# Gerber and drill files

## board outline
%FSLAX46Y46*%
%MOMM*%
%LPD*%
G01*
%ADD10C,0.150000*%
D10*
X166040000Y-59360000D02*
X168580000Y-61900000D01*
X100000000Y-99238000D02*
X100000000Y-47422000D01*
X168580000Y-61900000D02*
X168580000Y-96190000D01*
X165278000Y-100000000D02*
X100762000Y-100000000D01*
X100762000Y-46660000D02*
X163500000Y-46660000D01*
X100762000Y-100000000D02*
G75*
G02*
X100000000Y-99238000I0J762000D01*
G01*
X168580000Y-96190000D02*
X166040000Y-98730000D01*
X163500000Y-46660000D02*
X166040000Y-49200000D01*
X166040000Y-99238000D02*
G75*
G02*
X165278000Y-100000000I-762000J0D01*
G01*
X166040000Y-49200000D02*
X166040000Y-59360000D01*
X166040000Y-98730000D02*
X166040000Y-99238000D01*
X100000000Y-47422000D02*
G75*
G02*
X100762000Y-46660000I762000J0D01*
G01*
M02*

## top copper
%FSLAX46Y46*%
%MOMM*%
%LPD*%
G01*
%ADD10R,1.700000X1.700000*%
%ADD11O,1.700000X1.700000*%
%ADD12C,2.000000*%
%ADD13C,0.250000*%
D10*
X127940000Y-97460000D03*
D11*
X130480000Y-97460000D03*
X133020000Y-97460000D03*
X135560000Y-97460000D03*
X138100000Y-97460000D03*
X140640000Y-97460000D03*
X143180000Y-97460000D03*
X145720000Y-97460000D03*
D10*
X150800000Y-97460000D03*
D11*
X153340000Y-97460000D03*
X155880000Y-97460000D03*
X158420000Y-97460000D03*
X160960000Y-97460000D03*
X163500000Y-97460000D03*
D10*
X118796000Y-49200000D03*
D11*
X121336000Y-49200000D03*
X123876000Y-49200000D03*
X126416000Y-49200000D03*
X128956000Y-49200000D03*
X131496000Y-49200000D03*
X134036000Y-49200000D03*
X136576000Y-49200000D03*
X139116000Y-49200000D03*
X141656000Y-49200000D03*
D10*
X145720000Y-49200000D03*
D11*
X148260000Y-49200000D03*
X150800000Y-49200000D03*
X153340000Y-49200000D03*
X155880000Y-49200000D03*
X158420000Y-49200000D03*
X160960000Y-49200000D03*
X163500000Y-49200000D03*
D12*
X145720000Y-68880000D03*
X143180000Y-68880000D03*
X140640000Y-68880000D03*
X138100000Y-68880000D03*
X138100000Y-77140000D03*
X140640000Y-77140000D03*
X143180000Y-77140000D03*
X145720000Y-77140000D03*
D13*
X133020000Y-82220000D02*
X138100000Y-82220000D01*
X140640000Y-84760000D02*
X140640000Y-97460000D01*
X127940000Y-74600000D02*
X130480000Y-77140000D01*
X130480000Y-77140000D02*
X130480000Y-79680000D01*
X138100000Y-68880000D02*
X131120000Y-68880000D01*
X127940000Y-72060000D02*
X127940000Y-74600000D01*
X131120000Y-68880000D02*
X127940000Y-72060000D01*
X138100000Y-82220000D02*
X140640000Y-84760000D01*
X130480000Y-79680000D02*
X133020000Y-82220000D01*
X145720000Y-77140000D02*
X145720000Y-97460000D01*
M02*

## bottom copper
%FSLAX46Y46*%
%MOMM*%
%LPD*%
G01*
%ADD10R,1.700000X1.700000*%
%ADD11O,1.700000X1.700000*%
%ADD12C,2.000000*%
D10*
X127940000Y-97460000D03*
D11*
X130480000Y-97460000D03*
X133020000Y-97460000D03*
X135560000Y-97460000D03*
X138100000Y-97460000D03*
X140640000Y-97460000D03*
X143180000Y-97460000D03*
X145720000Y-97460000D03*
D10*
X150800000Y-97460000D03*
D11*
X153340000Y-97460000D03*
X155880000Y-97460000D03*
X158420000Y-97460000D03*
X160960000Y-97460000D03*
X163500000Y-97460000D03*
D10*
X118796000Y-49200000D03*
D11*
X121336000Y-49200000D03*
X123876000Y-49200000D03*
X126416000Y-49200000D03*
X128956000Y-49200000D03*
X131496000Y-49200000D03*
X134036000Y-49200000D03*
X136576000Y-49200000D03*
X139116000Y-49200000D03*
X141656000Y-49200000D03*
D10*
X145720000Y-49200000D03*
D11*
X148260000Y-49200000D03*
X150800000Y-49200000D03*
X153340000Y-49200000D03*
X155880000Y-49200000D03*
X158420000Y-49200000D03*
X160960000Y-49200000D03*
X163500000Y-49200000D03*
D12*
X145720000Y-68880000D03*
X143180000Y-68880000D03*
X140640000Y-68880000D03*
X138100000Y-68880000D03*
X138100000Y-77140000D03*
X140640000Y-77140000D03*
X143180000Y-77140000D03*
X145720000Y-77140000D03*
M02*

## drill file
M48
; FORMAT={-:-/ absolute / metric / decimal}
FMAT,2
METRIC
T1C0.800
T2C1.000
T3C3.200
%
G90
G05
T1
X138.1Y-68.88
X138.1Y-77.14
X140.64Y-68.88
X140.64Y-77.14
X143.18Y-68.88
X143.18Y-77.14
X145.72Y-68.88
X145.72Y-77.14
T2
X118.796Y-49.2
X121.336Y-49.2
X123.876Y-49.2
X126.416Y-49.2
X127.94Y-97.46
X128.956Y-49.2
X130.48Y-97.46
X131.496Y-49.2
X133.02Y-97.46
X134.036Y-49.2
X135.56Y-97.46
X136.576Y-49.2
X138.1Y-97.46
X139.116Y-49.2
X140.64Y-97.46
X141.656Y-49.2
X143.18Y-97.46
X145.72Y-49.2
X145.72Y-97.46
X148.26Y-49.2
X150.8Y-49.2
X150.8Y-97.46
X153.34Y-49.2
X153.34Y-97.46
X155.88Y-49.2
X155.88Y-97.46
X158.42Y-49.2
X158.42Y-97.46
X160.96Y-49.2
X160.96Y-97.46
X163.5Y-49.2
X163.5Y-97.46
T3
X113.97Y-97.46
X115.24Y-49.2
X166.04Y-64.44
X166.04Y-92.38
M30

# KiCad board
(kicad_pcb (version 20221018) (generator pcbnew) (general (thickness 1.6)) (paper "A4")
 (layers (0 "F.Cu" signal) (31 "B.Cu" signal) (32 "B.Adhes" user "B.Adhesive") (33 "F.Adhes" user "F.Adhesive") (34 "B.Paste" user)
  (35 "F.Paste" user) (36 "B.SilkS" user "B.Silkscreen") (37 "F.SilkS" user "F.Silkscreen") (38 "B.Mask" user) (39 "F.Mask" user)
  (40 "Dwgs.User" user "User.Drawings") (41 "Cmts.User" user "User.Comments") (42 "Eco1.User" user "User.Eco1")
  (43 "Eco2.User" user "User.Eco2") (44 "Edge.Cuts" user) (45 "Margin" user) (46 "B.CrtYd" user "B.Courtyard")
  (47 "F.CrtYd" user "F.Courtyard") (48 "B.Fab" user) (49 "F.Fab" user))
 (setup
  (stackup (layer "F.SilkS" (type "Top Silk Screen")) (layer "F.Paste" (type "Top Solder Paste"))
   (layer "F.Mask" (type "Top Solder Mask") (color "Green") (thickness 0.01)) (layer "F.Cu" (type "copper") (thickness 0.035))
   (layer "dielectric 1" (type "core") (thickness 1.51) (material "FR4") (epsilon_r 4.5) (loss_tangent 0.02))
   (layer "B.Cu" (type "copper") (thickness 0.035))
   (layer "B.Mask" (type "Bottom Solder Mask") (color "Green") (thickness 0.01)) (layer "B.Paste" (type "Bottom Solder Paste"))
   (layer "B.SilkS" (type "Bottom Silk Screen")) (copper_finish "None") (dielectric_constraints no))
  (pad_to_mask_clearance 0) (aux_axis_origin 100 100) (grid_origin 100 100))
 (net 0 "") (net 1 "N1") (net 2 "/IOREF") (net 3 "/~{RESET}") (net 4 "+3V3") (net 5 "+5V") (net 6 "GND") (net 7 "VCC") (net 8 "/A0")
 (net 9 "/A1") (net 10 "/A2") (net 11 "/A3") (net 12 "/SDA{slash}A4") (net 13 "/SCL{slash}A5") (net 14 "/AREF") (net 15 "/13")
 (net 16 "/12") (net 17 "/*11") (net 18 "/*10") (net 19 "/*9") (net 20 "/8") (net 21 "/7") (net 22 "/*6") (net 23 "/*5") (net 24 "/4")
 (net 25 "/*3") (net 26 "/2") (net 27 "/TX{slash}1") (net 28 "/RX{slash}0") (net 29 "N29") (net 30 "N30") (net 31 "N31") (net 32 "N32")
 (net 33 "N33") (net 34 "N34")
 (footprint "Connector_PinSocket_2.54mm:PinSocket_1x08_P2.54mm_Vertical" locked (layer "F.Cu") (at 127.94 97.46 90)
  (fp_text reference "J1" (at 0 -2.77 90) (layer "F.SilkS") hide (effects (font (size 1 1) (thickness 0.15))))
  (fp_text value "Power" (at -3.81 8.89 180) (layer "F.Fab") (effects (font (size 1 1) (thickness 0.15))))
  (pad "1" thru_hole rect locked (at 0 0 90) (size 1.7 1.7) (drill 1) (layers "*.Cu" "*.Mask") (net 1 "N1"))
  (pad "2" thru_hole oval locked (at 0 2.54 90) (size 1.7 1.7) (drill 1) (layers "*.Cu" "*.Mask") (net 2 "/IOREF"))
  (pad "3" thru_hole oval locked (at 0 5.08 90) (size 1.7 1.7) (drill 1) (layers "*.Cu" "*.Mask") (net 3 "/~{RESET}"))
  (pad "4" thru_hole oval locked (at 0 7.62 90) (size 1.7 1.7) (drill 1) (layers "*.Cu" "*.Mask") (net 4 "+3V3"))
  (pad "5" thru_hole oval locked (at 0 10.16 90) (size 1.7 1.7) (drill 1) (layers "*.Cu" "*.Mask") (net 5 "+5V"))
  (pad "6" thru_hole oval locked (at 0 12.7 90) (size 1.7 1.7) (drill 1) (layers "*.Cu" "*.Mask") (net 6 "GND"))
  (pad "7" thru_hole oval locked (at 0 15.24 90) (size 1.7 1.7) (drill 1) (layers "*.Cu" "*.Mask") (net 6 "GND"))
  (pad "8" thru_hole oval locked (at 0 17.78 90) (size 1.7 1.7) (drill 1) (layers "*.Cu" "*.Mask") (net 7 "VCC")))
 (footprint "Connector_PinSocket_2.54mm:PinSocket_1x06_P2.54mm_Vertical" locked (layer "F.Cu") (at 150.8 97.46 90)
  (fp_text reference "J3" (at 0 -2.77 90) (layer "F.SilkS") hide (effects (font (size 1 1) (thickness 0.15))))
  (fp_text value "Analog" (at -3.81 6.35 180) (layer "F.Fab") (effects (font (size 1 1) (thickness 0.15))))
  (pad "1" thru_hole rect locked (at 0 0 90) (size 1.7 1.7) (drill 1) (layers "*.Cu" "*.Mask") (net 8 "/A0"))
  (pad "2" thru_hole oval locked (at 0 2.54 90) (size 1.7 1.7) (drill 1) (layers "*.Cu" "*.Mask") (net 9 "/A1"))
  (pad "3" thru_hole oval locked (at 0 5.08 90) (size 1.7 1.7) (drill 1) (layers "*.Cu" "*.Mask") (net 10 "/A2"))
  (pad "4" thru_hole oval locked (at 0 7.62 90) (size 1.7 1.7) (drill 1) (layers "*.Cu" "*.Mask") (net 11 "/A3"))
  (pad "5" thru_hole oval locked (at 0 10.16 90) (size 1.7 1.7) (drill 1) (layers "*.Cu" "*.Mask") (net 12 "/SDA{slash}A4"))
  (pad "6" thru_hole oval locked (at 0 12.7 90) (size 1.7 1.7) (drill 1) (layers "*.Cu" "*.Mask") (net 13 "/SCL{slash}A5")))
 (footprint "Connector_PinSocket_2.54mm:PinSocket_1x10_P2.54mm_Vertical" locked (layer "F.Cu") (at 118.796 49.2 90)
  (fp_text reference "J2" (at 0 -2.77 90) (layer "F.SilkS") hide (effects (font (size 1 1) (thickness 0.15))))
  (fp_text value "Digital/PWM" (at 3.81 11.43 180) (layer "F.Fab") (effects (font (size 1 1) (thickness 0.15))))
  (pad "1" thru_hole rect locked (at 0 0 90) (size 1.7 1.7) (drill 1) (layers "*.Cu" "*.Mask") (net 13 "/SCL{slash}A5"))
  (pad "2" thru_hole oval locked (at 0 2.54 90) (size 1.7 1.7) (drill 1) (layers "*.Cu" "*.Mask") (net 12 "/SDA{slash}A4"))
  (pad "3" thru_hole oval locked (at 0 5.08 90) (size 1.7 1.7) (drill 1) (layers "*.Cu" "*.Mask") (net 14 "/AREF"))
  (pad "4" thru_hole oval locked (at 0 7.62 90) (size 1.7 1.7) (drill 1) (layers "*.Cu" "*.Mask") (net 6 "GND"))
  (pad "5" thru_hole oval locked (at 0 10.16 90) (size 1.7 1.7) (drill 1) (layers "*.Cu" "*.Mask") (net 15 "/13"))
  (pad "6" thru_hole oval locked (at 0 12.7 90) (size 1.7 1.7) (drill 1) (layers "*.Cu" "*.Mask") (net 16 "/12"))
  (pad "7" thru_hole oval locked (at 0 15.24 90) (size 1.7 1.7) (drill 1) (layers "*.Cu" "*.Mask") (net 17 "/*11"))
  (pad "8" thru_hole oval locked (at 0 17.78 90) (size 1.7 1.7) (drill 1) (layers "*.Cu" "*.Mask") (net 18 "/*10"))
  (pad "9" thru_hole oval locked (at 0 20.32 90) (size 1.7 1.7) (drill 1) (layers "*.Cu" "*.Mask") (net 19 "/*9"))
  (pad "10" thru_hole oval locked (at 0 22.86 90) (size 1.7 1.7) (drill 1) (layers "*.Cu" "*.Mask") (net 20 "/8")))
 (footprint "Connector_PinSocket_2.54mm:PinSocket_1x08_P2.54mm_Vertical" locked (layer "F.Cu") (at 145.72 49.2 90)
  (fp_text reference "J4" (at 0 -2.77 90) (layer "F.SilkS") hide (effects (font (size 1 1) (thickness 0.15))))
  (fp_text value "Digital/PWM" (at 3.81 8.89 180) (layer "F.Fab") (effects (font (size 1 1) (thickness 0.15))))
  (pad "1" thru_hole rect locked (at 0 0 90) (size 1.7 1.7) (drill 1) (layers "*.Cu" "*.Mask") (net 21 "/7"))
  (pad "2" thru_hole oval locked (at 0 2.54 90) (size 1.7 1.7) (drill 1) (layers "*.Cu" "*.Mask") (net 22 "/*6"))
  (pad "3" thru_hole oval locked (at 0 5.08 90) (size 1.7 1.7) (drill 1) (layers "*.Cu" "*.Mask") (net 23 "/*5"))
  (pad "4" thru_hole oval locked (at 0 7.62 90) (size 1.7 1.7) (drill 1) (layers "*.Cu" "*.Mask") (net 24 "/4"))
  (pad "5" thru_hole oval locked (at 0 10.16 90) (size 1.7 1.7) (drill 1) (layers "*.Cu" "*.Mask") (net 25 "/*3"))
  (pad "6" thru_hole oval locked (at 0 12.7 90) (size 1.7 1.7) (drill 1) (layers "*.Cu" "*.Mask") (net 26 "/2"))
  (pad "7" thru_hole oval locked (at 0 15.24 90) (size 1.7 1.7) (drill 1) (layers "*.Cu" "*.Mask") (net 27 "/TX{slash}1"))
  (pad "8" thru_hole oval locked (at 0 17.78 90) (size 1.7 1.7) (drill 1) (layers "*.Cu" "*.Mask") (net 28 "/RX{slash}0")))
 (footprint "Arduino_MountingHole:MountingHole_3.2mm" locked (layer "F.Cu") (at 115.24 49.2)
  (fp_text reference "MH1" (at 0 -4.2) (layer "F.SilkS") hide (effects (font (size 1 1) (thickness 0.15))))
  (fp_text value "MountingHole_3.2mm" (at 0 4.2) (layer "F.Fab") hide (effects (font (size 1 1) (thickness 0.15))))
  (pad "" np_thru_hole circle locked (at 0 0) (size 3.2 3.2) (drill 3.2) (layers "*.Cu" "*.Mask")))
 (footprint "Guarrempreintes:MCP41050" (layer "F.Cu") (at 141.91 72.64 180)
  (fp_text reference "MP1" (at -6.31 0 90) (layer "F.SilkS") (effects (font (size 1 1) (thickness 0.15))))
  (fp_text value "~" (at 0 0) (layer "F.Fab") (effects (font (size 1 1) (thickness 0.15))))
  (pad "1" thru_hole circle (at -3.81 3.76 180) (size 2 2) (drill 0.8) (layers "*.Cu" "*.Mask") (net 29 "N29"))
  (pad "2" thru_hole circle (at -1.27 3.76 180) (size 2 2) (drill 0.8) (layers "*.Cu" "*.Mask") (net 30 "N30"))
  (pad "3" thru_hole circle (at 1.27 3.76 180) (size 2 2) (drill 0.8) (layers "*.Cu" "*.Mask") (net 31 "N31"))
  (pad "4" thru_hole circle (at 3.81 3.76 180) (size 2 2) (drill 0.8) (layers "*.Cu" "*.Mask") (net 6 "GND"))
  (pad "5" thru_hole circle (at 3.81 -4.5 180) (size 2 2) (drill 0.8) (layers "*.Cu" "*.Mask") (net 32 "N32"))
  (pad "6" thru_hole circle (at 1.27 -4.5 180) (size 2 2) (drill 0.8) (layers "*.Cu" "*.Mask") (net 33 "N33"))
  (pad "7" thru_hole circle (at -1.27 -4.5 180) (size 2 2) (drill 0.8) (layers "*.Cu" "*.Mask") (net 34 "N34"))
  (pad "8" thru_hole circle (at -3.81 -4.5 180) (size 2 2) (drill 0.8) (layers "*.Cu" "*.Mask") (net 7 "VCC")))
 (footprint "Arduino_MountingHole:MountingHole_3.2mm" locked (layer "F.Cu") (at 113.97 97.46)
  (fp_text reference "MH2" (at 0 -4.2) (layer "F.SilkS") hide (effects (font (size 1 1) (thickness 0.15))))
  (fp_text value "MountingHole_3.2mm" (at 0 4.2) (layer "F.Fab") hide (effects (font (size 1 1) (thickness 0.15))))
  (pad "" np_thru_hole circle locked (at 0 0) (size 3.2 3.2) (drill 3.2) (layers "*.Cu" "*.Mask")))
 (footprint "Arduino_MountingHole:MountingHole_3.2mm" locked (layer "F.Cu") (at 166.04 64.44)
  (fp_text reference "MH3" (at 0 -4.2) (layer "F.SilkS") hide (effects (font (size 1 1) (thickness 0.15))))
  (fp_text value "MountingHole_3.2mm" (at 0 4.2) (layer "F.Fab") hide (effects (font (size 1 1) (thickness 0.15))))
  (pad "" np_thru_hole circle locked (at 0 0) (size 3.2 3.2) (drill 3.2) (layers "*.Cu" "*.Mask")))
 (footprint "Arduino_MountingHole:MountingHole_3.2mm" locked (layer "F.Cu") (at 166.04 92.38)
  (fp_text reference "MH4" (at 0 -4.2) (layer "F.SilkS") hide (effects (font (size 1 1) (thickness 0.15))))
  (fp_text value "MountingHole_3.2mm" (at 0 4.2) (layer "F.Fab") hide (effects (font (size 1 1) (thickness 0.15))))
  (pad "" np_thru_hole circle locked (at 0 0) (size 3.2 3.2) (drill 3.2) (layers "*.Cu" "*.Mask")))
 (gr_line (start 166.04 59.36) (end 168.58 61.9) (stroke (width 0.15) (type solid)) (layer "Edge.Cuts"))
 (gr_line (start 100 99.238) (end 100 47.422) (stroke (width 0.15) (type solid)) (layer "Edge.Cuts"))
 (gr_line (start 168.58 61.9) (end 168.58 96.19) (stroke (width 0.15) (type solid)) (layer "Edge.Cuts"))
 (gr_line (start 165.278 100) (end 100.762 100) (stroke (width 0.15) (type solid)) (layer "Edge.Cuts"))
 (gr_line (start 100.762 46.66) (end 163.5 46.66) (stroke (width 0.15) (type solid)) (layer "Edge.Cuts"))
 (gr_arc (start 100.762 100) (mid 100.223185 99.776815) (end 100 99.238) (stroke (width 0.15) (type solid)) (layer "Edge.Cuts"))
 (gr_line (start 168.58 96.19) (end 166.04 98.73) (stroke (width 0.15) (type solid)) (layer "Edge.Cuts"))
 (gr_line (start 163.5 46.66) (end 166.04 49.2) (stroke (width 0.15) (type solid)) (layer "Edge.Cuts"))
 (gr_arc (start 166.04 99.238) (mid 165.816815 99.776815) (end 165.278 100) (stroke (width 0.15) (type solid)) (layer "Edge.Cuts"))
 (gr_line (start 166.04 49.2) (end 166.04 59.36) (stroke (width 0.15) (type solid)) (layer "Edge.Cuts"))
 (gr_line (start 166.04 98.73) (end 166.04 99.238) (stroke (width 0.15) (type solid)) (layer "Edge.Cuts"))
 (gr_arc (start 100 47.422) (mid 100.223185 46.883185) (end 100.762 46.66) (stroke (width 0.15) (type solid)) (layer "Edge.Cuts"))
 (segment (start 133.02 82.22) (end 138.1 82.22) (width 0.25) (layer "F.Cu") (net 6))
 (segment (start 140.64 84.76) (end 140.64 97.46) (width 0.25) (layer "F.Cu") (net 6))
 (segment (start 127.94 74.6) (end 130.48 77.14) (width 0.25) (layer "F.Cu") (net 6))
 (segment (start 130.48 77.14) (end 130.48 79.68) (width 0.25) (layer "F.Cu") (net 6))
 (segment (start 138.1 68.88) (end 131.12 68.88) (width 0.25) (layer "F.Cu") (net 6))
 (segment (start 127.94 72.06) (end 127.94 74.6) (width 0.25) (layer "F.Cu") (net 6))
 (segment (start 131.12 68.88) (end 127.94 72.06) (width 0.25) (layer "F.Cu") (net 6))
 (segment (start 138.1 82.22) (end 140.64 84.76) (width 0.25) (layer "F.Cu") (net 6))
 (segment (start 130.48 79.68) (end 133.02 82.22) (width 0.25) (layer "F.Cu") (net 6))
 (segment (start 145.72 77.14) (end 145.72 97.46) (width 0.25) (layer "F.Cu") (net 7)))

